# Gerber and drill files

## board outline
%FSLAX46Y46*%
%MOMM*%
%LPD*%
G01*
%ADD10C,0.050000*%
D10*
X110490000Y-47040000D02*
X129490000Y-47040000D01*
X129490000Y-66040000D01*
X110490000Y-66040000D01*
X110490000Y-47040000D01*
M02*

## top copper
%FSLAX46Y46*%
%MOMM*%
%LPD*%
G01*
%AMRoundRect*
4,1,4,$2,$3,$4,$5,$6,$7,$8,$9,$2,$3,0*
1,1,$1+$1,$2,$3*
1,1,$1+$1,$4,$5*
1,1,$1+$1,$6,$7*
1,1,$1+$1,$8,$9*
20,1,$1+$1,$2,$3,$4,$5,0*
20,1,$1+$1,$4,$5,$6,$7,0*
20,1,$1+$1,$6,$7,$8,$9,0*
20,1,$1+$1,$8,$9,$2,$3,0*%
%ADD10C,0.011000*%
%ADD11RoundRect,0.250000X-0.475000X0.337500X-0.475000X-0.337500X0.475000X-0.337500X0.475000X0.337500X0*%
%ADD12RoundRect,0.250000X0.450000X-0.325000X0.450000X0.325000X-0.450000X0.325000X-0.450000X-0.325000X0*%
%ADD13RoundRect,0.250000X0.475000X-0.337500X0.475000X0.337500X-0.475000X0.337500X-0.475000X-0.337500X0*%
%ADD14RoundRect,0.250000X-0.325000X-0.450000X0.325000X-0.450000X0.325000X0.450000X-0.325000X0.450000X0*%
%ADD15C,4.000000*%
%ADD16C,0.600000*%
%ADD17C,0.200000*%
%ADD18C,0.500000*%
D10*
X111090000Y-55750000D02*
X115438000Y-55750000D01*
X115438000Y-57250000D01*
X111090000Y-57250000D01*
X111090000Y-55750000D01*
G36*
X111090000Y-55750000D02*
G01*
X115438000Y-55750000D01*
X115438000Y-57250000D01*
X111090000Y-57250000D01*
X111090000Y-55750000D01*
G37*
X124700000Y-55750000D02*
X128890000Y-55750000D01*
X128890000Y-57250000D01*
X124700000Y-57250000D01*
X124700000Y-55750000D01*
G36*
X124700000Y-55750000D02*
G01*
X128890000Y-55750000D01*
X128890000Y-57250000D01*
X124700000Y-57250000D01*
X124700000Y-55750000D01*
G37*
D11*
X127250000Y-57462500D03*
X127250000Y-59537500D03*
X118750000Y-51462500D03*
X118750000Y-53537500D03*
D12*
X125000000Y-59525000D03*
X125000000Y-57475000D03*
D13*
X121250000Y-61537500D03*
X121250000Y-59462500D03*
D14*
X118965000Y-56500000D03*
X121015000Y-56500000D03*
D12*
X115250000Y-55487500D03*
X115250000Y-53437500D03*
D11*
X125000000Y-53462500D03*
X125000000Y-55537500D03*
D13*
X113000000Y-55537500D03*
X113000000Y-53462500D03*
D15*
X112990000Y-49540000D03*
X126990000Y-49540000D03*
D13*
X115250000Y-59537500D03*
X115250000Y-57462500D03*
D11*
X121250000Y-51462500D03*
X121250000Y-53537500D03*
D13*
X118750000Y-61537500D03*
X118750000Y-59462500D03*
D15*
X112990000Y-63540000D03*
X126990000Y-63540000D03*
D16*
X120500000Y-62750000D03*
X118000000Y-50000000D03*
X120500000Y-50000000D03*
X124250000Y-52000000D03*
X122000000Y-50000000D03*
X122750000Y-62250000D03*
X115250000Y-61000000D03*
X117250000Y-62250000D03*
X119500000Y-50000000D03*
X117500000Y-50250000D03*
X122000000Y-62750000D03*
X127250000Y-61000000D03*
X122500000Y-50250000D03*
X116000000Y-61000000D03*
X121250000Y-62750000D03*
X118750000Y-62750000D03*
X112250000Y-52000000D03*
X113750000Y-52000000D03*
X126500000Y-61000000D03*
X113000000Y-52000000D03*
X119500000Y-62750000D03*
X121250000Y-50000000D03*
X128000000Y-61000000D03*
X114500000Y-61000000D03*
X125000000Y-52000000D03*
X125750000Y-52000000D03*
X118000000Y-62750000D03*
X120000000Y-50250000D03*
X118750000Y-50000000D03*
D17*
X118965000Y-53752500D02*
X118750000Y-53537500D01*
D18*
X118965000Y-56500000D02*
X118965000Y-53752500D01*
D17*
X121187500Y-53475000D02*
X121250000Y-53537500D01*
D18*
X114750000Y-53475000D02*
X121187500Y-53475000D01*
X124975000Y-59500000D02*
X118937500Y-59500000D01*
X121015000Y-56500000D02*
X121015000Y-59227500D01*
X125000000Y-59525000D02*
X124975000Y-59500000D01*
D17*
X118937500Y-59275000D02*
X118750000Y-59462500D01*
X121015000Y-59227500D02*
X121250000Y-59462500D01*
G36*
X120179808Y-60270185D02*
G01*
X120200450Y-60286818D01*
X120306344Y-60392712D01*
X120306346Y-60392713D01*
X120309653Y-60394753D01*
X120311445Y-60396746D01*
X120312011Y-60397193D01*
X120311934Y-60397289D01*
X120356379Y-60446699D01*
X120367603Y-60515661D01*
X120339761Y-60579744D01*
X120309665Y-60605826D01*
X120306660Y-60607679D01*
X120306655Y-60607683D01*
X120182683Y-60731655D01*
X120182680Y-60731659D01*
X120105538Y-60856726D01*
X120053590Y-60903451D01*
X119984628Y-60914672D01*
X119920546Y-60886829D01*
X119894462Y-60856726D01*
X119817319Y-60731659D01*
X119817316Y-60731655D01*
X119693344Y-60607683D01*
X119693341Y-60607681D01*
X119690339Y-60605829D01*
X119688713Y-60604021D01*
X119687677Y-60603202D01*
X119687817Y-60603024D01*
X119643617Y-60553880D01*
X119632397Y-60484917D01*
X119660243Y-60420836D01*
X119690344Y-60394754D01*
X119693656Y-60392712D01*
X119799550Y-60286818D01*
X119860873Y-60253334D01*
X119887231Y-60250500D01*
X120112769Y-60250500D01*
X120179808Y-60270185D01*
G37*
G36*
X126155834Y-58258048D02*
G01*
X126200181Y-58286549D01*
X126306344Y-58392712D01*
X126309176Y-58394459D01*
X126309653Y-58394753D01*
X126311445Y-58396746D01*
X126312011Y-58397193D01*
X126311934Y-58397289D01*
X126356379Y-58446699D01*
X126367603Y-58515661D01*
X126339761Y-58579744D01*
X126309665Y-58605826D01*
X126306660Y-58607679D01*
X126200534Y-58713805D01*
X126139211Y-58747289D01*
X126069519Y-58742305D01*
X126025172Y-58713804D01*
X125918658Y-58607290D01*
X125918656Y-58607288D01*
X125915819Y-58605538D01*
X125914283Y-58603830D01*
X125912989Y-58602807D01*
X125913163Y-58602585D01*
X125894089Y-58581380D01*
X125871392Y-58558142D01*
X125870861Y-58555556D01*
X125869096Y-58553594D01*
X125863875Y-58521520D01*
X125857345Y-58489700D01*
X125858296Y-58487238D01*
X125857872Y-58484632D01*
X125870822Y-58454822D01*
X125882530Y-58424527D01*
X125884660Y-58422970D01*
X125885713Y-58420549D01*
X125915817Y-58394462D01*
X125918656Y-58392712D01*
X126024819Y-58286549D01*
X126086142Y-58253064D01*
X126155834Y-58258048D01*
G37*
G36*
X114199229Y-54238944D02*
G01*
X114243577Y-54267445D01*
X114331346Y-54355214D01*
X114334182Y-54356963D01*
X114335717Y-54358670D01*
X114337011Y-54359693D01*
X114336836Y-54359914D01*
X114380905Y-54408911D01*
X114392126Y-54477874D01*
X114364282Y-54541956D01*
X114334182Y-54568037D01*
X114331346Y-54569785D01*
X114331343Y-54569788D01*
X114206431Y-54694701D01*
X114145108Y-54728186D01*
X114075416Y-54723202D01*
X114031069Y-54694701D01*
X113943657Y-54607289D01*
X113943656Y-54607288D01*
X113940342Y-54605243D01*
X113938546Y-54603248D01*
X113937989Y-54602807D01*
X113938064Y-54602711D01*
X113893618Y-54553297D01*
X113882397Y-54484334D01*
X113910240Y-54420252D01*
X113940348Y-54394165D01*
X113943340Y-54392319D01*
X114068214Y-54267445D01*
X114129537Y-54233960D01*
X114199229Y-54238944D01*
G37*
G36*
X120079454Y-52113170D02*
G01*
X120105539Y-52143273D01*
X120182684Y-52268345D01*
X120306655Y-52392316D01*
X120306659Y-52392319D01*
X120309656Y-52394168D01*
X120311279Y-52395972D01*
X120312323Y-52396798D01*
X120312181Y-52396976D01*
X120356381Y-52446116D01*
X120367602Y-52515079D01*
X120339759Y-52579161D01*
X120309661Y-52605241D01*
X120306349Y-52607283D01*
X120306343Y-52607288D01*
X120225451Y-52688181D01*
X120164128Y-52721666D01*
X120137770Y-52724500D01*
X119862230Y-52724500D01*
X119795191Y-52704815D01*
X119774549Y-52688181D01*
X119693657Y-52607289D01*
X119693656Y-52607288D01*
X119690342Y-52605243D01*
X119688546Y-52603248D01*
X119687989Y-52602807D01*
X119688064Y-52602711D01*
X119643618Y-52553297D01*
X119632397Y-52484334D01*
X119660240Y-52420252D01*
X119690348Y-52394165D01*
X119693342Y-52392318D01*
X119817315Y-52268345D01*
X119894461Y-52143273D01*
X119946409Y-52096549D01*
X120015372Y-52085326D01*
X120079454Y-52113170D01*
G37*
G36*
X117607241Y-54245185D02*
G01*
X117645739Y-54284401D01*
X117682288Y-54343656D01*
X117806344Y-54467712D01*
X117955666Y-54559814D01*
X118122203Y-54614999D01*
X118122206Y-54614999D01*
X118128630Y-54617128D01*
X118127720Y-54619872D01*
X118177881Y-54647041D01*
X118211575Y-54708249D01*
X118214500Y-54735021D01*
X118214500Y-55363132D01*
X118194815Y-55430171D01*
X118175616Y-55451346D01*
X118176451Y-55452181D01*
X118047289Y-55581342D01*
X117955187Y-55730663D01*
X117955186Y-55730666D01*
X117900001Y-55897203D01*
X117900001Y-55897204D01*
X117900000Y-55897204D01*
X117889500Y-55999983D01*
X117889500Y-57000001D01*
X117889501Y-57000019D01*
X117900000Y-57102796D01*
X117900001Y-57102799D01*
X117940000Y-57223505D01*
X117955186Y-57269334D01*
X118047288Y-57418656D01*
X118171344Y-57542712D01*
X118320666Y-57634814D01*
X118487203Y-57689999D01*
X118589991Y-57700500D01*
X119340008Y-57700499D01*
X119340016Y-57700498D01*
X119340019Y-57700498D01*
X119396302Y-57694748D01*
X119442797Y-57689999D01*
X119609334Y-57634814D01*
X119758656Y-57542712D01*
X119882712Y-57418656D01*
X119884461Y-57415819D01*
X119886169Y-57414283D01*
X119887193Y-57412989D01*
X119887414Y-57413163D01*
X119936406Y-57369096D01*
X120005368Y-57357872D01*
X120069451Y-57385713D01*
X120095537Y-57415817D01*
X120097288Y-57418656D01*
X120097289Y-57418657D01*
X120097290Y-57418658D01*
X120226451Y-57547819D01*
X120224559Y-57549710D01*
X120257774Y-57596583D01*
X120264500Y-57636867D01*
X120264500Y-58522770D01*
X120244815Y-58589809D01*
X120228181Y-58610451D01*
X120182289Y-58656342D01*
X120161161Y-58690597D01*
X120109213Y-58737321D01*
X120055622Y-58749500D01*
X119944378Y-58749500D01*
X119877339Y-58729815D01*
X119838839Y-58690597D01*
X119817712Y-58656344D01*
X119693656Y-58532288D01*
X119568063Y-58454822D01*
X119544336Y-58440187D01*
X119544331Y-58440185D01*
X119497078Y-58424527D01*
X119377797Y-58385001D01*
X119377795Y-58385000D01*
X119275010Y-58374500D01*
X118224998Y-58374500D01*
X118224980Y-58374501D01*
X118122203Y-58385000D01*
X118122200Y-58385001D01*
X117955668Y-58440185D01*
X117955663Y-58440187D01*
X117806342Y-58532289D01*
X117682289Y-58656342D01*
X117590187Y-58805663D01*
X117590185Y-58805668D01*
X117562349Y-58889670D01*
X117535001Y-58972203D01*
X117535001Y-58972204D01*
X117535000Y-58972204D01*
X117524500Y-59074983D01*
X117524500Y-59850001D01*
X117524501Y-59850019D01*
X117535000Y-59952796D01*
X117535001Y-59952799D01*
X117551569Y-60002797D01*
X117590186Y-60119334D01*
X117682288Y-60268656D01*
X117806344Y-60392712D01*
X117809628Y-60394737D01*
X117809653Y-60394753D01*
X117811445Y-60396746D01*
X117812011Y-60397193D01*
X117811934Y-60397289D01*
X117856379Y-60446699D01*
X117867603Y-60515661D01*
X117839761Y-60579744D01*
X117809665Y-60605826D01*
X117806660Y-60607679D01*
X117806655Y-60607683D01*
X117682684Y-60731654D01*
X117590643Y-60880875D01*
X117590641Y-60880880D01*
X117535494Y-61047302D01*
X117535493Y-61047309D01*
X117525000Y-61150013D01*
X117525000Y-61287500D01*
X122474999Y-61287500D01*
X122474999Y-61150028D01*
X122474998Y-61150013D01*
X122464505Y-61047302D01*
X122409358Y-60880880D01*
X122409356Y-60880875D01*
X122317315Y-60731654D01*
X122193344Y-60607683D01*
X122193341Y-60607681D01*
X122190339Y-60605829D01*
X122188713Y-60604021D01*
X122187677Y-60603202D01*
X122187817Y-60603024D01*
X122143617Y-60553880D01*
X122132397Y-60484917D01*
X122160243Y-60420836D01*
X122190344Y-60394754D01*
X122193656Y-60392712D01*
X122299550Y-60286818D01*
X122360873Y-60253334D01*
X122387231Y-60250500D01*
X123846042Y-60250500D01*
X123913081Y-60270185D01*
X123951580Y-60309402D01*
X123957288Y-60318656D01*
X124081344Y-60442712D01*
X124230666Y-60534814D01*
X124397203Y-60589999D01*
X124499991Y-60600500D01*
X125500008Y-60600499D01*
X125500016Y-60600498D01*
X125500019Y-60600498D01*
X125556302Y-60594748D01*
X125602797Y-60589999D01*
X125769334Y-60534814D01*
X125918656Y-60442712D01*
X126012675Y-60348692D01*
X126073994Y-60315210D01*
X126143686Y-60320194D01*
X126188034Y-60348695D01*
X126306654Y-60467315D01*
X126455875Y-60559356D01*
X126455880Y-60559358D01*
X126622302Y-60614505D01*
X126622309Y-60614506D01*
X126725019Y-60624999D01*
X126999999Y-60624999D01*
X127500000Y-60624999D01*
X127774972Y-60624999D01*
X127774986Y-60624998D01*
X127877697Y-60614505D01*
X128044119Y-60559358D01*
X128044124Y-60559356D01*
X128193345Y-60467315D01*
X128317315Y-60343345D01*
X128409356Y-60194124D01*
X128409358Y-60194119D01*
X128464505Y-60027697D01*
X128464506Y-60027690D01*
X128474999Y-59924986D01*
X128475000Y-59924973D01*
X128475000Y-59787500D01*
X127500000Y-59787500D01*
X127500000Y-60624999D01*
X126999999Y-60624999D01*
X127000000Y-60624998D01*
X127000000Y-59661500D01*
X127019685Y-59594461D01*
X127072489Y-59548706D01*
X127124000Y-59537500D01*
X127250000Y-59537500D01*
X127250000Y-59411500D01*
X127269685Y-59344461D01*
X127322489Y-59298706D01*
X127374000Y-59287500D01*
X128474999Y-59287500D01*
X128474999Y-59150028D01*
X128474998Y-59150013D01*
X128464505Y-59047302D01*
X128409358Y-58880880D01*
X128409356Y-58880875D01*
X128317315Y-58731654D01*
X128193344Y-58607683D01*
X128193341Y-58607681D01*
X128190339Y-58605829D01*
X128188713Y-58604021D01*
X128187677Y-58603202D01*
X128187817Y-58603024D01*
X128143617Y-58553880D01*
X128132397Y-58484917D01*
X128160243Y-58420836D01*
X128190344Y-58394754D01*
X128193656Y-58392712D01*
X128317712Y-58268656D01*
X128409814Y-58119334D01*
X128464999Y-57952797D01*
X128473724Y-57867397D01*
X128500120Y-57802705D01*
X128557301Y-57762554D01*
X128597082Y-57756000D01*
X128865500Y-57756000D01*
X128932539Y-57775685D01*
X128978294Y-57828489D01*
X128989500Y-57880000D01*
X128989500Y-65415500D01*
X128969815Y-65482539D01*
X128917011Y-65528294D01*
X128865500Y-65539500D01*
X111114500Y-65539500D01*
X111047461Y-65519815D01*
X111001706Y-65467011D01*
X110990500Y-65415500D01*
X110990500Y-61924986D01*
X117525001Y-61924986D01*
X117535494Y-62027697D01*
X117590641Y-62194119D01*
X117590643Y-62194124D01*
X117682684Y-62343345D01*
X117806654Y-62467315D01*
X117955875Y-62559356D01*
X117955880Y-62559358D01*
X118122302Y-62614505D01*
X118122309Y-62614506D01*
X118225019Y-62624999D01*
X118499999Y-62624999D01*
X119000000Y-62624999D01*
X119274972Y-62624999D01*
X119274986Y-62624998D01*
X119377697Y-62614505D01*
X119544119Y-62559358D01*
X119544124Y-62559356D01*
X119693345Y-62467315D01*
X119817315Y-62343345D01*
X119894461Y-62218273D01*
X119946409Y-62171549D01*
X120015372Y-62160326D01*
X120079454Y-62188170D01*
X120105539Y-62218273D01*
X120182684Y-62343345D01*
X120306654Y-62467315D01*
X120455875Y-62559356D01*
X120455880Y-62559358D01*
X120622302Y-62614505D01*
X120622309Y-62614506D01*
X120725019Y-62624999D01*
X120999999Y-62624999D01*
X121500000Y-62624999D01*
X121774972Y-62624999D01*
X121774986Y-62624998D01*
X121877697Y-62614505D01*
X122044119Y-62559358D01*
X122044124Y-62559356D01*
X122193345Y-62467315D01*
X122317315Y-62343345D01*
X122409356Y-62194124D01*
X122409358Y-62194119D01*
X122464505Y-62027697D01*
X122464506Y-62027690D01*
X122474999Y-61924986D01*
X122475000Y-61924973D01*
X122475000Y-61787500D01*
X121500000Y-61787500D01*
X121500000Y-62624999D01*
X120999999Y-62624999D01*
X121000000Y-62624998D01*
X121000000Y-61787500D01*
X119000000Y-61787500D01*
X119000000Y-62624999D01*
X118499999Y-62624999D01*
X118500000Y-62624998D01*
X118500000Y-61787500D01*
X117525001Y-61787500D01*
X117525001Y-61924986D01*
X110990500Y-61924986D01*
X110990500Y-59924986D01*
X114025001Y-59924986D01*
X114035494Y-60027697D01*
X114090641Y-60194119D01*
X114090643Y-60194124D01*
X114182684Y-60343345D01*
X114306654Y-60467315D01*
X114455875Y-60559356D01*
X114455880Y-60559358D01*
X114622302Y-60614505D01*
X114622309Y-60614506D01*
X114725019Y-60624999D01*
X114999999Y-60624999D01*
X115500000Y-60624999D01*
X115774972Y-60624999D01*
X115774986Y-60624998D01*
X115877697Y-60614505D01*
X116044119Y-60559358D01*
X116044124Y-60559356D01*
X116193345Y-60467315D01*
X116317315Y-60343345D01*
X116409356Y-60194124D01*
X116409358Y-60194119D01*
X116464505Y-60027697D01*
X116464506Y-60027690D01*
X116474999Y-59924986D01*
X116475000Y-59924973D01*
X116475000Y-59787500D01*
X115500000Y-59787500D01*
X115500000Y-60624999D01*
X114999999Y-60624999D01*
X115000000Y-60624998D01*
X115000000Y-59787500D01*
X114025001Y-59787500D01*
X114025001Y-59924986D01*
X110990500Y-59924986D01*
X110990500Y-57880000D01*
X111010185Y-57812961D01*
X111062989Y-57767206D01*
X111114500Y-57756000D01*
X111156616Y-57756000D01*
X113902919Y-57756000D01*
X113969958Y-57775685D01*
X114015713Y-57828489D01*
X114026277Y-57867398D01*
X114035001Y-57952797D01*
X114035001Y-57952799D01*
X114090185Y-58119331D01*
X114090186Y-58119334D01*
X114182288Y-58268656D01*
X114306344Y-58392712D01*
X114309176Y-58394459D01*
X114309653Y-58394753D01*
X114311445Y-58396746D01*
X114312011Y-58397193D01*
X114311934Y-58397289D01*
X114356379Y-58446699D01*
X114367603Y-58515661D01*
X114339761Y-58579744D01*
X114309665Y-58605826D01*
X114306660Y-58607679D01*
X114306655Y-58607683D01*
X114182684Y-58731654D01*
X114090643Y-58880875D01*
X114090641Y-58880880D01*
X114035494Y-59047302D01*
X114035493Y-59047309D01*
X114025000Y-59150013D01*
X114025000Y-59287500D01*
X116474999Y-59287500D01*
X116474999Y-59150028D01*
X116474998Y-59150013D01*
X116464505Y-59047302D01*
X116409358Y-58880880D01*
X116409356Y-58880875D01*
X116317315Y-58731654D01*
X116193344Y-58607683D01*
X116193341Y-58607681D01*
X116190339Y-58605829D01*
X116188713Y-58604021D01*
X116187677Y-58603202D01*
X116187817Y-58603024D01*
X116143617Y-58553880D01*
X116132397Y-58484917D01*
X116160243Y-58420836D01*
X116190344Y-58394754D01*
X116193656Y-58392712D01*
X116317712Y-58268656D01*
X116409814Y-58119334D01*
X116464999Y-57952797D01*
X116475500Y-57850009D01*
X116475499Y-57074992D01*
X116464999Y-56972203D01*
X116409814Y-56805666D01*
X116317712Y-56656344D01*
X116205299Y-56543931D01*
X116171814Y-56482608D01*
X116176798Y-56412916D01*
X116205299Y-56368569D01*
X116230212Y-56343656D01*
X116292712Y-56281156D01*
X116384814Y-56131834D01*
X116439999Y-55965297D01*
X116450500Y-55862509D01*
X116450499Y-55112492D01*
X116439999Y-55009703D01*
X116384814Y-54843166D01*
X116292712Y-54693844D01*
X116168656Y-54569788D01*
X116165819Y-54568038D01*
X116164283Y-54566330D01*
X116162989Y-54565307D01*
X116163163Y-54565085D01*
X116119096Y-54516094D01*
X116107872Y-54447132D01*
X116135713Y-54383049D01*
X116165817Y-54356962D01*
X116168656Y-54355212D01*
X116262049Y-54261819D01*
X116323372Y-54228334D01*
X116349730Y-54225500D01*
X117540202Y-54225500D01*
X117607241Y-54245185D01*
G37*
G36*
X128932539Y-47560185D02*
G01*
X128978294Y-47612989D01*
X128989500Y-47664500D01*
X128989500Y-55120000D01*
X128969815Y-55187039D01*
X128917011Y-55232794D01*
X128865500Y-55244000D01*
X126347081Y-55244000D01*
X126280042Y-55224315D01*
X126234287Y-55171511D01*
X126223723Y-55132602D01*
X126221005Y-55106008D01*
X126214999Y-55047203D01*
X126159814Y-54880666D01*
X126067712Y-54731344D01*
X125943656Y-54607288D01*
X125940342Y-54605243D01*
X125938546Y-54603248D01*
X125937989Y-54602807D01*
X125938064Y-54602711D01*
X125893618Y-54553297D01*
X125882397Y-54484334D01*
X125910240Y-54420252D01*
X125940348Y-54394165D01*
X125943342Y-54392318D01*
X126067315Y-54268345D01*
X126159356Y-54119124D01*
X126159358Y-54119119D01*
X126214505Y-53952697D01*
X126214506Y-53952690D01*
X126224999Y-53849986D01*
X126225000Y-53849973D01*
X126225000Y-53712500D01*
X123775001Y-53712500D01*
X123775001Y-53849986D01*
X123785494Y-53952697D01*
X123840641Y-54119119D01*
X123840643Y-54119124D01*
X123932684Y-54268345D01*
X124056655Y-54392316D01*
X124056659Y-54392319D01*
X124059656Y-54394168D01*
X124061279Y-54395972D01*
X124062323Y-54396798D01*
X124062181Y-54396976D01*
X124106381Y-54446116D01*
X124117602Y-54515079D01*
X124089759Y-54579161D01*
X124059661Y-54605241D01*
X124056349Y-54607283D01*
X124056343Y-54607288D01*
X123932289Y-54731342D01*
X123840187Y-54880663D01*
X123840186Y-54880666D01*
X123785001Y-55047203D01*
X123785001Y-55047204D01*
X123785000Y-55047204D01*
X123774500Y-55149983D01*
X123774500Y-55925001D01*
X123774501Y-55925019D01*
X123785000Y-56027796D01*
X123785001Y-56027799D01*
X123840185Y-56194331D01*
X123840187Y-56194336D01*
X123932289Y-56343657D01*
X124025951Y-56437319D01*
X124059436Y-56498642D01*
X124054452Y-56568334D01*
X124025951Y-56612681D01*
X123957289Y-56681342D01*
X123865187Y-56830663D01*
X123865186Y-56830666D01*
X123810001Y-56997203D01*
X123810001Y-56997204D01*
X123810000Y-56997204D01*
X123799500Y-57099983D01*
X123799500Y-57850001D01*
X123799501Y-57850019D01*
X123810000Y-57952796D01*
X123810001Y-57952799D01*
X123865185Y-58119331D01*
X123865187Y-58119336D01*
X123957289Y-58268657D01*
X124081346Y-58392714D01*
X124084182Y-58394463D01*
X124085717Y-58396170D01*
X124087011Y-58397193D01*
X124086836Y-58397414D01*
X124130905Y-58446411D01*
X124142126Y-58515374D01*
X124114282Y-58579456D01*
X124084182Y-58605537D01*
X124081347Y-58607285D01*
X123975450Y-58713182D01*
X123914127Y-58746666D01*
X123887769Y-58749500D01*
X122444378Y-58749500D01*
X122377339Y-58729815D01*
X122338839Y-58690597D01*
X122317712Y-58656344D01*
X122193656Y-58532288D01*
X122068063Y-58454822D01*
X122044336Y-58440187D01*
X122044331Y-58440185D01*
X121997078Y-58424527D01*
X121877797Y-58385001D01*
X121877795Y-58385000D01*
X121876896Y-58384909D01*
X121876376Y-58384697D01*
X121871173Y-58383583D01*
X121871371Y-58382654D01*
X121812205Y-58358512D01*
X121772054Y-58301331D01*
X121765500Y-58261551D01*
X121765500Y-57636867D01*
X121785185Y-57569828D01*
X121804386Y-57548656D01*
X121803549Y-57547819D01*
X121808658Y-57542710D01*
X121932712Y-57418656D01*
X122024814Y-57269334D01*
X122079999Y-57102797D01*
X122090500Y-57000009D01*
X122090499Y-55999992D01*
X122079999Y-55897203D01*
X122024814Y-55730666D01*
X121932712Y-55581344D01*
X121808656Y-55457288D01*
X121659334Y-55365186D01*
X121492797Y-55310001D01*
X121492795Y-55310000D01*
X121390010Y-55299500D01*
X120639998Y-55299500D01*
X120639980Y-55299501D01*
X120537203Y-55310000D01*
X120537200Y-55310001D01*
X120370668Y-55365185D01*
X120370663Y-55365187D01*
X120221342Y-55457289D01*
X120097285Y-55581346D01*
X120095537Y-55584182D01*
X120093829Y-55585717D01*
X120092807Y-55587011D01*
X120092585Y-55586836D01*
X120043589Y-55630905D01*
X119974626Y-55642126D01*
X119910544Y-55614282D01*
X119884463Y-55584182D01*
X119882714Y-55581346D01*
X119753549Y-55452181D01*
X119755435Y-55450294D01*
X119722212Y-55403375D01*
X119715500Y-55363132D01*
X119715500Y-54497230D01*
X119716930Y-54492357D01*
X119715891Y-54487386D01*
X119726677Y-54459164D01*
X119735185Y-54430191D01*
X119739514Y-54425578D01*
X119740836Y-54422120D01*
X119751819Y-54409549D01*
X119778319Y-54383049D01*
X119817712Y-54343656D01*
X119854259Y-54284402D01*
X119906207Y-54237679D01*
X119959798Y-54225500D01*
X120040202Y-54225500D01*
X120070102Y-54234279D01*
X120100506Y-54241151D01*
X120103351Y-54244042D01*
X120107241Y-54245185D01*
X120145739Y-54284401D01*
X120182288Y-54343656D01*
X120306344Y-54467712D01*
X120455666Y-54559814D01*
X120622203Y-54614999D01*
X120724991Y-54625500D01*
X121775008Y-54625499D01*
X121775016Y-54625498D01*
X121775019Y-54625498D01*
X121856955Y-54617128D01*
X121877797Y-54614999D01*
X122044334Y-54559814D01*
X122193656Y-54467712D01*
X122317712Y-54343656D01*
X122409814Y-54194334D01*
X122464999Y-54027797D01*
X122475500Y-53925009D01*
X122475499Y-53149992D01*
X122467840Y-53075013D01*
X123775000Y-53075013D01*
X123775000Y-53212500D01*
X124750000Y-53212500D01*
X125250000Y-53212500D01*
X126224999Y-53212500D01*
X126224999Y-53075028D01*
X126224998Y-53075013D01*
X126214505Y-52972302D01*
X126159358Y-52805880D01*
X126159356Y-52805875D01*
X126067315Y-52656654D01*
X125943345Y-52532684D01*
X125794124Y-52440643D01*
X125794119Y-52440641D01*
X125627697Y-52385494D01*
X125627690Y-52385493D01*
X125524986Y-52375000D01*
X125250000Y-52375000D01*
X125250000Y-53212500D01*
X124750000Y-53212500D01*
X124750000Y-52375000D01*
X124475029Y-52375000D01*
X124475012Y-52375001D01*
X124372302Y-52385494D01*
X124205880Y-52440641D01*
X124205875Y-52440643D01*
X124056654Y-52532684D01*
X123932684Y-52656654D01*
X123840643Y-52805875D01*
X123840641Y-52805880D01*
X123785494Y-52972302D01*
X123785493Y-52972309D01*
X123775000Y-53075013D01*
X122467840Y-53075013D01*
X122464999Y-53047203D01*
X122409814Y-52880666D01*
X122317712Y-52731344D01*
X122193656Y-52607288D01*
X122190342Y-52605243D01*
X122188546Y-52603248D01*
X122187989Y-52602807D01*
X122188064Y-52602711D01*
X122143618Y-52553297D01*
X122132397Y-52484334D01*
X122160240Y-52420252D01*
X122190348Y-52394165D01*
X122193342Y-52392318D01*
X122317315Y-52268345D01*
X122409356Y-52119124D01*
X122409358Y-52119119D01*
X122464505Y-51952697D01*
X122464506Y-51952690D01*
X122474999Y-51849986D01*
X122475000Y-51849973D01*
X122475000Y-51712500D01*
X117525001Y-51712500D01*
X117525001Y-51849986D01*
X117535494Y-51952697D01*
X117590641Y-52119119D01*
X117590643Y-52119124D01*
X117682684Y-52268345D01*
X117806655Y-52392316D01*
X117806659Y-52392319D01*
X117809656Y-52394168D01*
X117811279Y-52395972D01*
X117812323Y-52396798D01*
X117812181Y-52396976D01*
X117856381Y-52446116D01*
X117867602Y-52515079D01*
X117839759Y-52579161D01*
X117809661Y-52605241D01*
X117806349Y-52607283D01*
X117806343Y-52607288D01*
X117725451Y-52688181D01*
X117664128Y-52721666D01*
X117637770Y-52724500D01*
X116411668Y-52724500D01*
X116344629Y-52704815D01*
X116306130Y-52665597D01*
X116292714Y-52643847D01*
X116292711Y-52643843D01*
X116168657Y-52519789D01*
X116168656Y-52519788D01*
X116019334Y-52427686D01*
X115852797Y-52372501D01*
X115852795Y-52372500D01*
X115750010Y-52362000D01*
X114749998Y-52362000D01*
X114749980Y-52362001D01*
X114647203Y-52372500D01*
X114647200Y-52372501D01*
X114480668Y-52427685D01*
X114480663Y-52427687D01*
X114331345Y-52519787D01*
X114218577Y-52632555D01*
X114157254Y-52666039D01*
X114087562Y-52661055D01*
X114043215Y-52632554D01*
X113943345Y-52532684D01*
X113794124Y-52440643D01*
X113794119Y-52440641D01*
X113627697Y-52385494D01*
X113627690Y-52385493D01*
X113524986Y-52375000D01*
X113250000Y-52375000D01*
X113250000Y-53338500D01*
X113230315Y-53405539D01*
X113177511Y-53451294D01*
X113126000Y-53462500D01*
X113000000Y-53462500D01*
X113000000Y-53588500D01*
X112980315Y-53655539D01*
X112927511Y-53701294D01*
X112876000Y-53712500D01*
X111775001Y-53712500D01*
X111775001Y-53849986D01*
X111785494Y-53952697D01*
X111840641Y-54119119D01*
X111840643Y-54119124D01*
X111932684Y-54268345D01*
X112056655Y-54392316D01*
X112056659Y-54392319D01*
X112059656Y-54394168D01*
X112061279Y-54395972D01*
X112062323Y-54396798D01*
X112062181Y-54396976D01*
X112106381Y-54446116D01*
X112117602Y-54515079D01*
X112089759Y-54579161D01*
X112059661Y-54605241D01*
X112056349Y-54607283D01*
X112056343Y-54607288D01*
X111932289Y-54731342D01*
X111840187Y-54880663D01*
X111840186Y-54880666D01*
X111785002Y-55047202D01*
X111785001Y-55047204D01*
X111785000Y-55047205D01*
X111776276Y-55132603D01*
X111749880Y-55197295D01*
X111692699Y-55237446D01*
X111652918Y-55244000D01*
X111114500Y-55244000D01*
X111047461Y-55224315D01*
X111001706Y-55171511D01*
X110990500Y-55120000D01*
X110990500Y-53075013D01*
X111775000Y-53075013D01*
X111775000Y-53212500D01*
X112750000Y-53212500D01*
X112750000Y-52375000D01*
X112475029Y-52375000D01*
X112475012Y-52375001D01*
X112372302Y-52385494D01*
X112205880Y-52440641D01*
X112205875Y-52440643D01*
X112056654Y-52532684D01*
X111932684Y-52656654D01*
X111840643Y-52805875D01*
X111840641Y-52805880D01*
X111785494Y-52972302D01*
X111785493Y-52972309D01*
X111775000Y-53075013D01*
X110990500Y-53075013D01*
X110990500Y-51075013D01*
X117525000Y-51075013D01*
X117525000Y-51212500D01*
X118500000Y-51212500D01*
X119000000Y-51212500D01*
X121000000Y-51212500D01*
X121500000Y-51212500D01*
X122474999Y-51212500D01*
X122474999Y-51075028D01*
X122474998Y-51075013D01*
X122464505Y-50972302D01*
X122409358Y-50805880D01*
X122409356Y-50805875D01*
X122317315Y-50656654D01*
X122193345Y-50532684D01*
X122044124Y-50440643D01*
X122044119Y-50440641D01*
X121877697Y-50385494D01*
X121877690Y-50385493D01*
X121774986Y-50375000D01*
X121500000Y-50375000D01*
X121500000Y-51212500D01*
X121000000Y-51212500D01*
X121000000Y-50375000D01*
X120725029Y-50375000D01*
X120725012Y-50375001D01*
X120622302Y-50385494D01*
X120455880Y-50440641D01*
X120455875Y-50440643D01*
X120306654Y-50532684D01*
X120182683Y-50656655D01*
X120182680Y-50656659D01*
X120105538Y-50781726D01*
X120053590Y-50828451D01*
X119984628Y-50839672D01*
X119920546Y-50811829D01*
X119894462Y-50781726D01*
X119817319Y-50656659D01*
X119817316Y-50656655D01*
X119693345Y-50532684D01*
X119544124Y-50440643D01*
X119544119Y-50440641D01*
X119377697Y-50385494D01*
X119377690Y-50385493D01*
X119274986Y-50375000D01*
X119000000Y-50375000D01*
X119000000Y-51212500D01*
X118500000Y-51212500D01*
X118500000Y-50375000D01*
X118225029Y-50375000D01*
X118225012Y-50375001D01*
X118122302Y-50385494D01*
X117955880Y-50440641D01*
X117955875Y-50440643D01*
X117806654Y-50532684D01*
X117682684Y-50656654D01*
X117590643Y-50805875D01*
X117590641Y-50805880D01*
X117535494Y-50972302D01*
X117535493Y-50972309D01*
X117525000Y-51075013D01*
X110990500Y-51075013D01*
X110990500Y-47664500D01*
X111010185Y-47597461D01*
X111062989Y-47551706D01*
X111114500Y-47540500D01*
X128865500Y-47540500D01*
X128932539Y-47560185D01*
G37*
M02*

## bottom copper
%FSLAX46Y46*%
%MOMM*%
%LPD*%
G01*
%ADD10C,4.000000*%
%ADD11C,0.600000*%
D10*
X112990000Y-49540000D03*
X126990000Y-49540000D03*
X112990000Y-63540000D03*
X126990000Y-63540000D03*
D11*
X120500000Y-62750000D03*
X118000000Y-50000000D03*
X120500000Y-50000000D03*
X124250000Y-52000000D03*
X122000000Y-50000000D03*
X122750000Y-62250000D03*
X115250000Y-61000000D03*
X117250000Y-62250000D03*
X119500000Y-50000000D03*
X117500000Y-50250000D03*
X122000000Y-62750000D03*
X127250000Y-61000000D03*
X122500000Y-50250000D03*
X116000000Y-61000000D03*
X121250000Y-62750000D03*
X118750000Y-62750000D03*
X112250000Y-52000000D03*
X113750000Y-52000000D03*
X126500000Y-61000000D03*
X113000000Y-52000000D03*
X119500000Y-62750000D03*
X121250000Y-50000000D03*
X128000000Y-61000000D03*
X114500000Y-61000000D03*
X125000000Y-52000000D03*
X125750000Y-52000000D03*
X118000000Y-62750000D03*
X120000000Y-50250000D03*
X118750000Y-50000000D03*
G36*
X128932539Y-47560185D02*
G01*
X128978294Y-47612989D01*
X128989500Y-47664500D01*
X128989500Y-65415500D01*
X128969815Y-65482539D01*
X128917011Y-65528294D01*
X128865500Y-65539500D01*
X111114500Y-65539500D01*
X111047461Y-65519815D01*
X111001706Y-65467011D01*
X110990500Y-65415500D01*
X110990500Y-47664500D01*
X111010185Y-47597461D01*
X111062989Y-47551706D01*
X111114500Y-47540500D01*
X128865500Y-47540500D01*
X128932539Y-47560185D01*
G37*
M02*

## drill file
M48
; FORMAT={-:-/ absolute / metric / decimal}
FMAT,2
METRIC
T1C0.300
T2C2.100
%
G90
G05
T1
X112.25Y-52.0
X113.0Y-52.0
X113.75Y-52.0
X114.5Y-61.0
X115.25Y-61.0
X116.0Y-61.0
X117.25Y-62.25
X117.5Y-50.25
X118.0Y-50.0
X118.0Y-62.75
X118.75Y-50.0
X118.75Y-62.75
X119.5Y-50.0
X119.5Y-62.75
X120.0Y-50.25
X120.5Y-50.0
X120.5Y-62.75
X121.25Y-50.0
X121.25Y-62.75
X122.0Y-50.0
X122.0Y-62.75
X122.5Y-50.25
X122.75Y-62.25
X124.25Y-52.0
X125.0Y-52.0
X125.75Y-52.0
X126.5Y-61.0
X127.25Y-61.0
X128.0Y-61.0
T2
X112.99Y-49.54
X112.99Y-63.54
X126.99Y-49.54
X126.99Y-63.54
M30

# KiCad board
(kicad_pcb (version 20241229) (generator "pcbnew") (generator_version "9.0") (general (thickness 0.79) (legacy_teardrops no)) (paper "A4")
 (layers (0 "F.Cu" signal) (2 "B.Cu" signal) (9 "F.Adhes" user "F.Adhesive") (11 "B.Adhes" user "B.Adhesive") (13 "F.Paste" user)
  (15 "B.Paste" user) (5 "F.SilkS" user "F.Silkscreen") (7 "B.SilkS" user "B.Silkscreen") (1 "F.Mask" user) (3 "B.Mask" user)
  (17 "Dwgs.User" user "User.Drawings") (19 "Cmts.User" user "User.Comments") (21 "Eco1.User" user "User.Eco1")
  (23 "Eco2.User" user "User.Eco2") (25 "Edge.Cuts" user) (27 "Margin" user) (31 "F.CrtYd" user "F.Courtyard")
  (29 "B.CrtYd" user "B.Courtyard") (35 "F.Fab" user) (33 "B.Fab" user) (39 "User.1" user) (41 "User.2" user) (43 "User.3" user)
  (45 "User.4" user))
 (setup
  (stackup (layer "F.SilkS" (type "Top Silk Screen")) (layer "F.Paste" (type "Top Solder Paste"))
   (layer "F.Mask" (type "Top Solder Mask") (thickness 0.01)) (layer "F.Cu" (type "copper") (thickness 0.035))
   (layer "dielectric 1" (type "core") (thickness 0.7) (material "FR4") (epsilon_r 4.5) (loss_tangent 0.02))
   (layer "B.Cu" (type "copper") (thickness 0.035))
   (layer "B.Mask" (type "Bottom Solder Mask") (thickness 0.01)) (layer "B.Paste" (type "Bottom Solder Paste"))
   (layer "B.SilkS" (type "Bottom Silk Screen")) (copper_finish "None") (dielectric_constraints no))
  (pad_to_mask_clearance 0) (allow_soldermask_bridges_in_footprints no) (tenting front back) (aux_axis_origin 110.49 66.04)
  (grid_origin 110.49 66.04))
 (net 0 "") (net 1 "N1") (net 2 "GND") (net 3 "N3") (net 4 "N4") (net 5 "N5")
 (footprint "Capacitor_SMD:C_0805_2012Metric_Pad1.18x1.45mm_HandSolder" (layer "F.Cu") (at 127.25 58.5 -90)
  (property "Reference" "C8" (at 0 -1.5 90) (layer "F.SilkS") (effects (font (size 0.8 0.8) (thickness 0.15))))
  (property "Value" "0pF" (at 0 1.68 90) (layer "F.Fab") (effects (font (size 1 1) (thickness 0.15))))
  (pad "1" smd roundrect (at -1.0375 0 270) (size 1.175 1.45) (layers "F.Cu" "F.Mask" "F.Paste") (roundrect_rratio 0.212766) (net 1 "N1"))
  (pad "2" smd roundrect (at 1.0375 0 270) (size 1.175 1.45) (layers "F.Cu" "F.Mask" "F.Paste") (roundrect_rratio 0.212766) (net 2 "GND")))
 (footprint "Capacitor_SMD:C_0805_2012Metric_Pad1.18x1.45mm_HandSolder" (layer "F.Cu") (at 118.75 52.5 -90)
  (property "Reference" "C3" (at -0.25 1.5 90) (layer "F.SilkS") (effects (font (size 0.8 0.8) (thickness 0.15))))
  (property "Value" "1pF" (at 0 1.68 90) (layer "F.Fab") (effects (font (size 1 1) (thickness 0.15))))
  (pad "1" smd roundrect (at -1.0375 0 270) (size 1.175 1.45) (layers "F.Cu" "F.Mask" "F.Paste") (roundrect_rratio 0.212766) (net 2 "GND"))
  (pad "2" smd roundrect (at 1.0375 0 270) (size 1.175 1.45) (layers "F.Cu" "F.Mask" "F.Paste") (roundrect_rratio 0.212766) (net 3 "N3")))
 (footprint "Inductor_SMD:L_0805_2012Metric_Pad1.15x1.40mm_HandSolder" (layer "F.Cu") (at 125 58.5 90)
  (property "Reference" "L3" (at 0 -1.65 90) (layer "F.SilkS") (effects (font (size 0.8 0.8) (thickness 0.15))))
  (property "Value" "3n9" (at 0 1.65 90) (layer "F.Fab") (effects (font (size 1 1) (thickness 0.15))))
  (pad "1" smd roundrect (at -1.025 0 90) (size 1.15 1.4) (layers "F.Cu" "F.Mask" "F.Paste") (roundrect_rratio 0.217391) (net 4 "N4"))
  (pad "2" smd roundrect (at 1.025 0 90) (size 1.15 1.4) (layers "F.Cu" "F.Mask" "F.Paste") (roundrect_rratio 0.217391) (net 1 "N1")))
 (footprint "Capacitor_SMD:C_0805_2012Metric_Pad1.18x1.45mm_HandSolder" (layer "F.Cu") (at 121.25 60.5 90)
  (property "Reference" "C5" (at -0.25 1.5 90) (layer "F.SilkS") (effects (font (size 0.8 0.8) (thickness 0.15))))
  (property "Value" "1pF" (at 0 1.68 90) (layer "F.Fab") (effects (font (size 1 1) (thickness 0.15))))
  (pad "1" smd roundrect (at -1.0375 0 90) (size 1.175 1.45) (layers "F.Cu" "F.Mask" "F.Paste") (roundrect_rratio 0.212766) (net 2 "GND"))
  (pad "2" smd roundrect (at 1.0375 0 90) (size 1.175 1.45) (layers "F.Cu" "F.Mask" "F.Paste") (roundrect_rratio 0.212766) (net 4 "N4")))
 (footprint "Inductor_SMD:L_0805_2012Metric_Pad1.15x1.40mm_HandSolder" (layer "F.Cu") (at 119.99 56.5)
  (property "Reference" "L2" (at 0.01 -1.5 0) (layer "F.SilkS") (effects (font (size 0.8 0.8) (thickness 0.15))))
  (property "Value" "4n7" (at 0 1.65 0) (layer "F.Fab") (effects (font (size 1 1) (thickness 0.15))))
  (pad "1" smd roundrect (at -1.025 0) (size 1.15 1.4) (layers "F.Cu" "F.Mask" "F.Paste") (roundrect_rratio 0.217391) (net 3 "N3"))
  (pad "2" smd roundrect (at 1.025 0) (size 1.15 1.4) (layers "F.Cu" "F.Mask" "F.Paste") (roundrect_rratio 0.217391) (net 4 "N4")))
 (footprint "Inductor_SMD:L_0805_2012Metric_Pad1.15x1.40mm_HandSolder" (layer "F.Cu") (at 115.25 54.4625 90)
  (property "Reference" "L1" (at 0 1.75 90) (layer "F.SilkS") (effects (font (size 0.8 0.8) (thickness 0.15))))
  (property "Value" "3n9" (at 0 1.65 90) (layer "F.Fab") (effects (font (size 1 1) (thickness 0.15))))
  (pad "1" smd roundrect (at -1.025 0 90) (size 1.15 1.4) (layers "F.Cu" "F.Mask" "F.Paste") (roundrect_rratio 0.217391) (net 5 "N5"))
  (pad "2" smd roundrect (at 1.025 0 90) (size 1.15 1.4) (layers "F.Cu" "F.Mask" "F.Paste") (roundrect_rratio 0.217391) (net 3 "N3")))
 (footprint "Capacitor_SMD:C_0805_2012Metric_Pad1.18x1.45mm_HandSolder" (layer "F.Cu") (at 125 54.5 -90)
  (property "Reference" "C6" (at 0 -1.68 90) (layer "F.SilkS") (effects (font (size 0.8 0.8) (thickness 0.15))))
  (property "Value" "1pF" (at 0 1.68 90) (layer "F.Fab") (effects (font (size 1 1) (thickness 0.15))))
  (pad "1" smd roundrect (at -1.0375 0 270) (size 1.175 1.45) (layers "F.Cu" "F.Mask" "F.Paste") (roundrect_rratio 0.212766) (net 2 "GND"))
  (pad "2" smd roundrect (at 1.0375 0 270) (size 1.175 1.45) (layers "F.Cu" "F.Mask" "F.Paste") (roundrect_rratio 0.212766) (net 1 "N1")))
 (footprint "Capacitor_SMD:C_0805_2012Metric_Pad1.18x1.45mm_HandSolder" (layer "F.Cu") (at 113 54.5 90)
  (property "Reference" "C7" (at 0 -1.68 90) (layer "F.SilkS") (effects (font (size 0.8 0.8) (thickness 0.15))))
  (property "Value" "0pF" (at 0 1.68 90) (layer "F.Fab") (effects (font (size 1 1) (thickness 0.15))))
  (pad "1" smd roundrect (at -1.0375 0 90) (size 1.175 1.45) (layers "F.Cu" "F.Mask" "F.Paste") (roundrect_rratio 0.212766) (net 5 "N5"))
  (pad "2" smd roundrect (at 1.0375 0 90) (size 1.175 1.45) (layers "F.Cu" "F.Mask" "F.Paste") (roundrect_rratio 0.212766) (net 2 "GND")))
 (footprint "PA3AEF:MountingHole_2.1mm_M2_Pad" (layer "F.Cu") (at 112.99 49.54)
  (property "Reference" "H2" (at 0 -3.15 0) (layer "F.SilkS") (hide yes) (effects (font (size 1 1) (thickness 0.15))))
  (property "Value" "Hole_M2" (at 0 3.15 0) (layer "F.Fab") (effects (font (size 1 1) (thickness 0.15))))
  (pad "1" thru_hole circle (at 0 0) (size 4 4) (drill 2.1) (layers "*.Cu" "*.Mask") (remove_unused_layers no) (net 2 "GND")
   (zone_connect 2)))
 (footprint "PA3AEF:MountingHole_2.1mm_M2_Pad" (layer "F.Cu") (at 126.99 49.54)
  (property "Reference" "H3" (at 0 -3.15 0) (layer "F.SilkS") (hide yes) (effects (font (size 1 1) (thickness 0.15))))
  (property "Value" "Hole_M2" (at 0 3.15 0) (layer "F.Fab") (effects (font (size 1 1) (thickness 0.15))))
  (pad "1" thru_hole circle (at 0 0) (size 4 4) (drill 2.1) (layers "*.Cu" "*.Mask") (remove_unused_layers no) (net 2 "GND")
   (zone_connect 2)))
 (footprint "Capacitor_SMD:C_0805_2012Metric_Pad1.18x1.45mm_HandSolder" (layer "F.Cu") (at 115.25 58.5 90)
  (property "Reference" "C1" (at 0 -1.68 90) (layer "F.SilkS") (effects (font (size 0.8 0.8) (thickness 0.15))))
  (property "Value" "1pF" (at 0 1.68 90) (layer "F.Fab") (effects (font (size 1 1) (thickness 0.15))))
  (pad "1" smd roundrect (at -1.0375 0 90) (size 1.175 1.45) (layers "F.Cu" "F.Mask" "F.Paste") (roundrect_rratio 0.212766) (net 2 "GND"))
  (pad "2" smd roundrect (at 1.0375 0 90) (size 1.175 1.45) (layers "F.Cu" "F.Mask" "F.Paste") (roundrect_rratio 0.212766) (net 5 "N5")))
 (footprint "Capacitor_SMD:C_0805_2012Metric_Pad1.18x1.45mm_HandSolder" (layer "F.Cu") (at 121.25 52.5 -90)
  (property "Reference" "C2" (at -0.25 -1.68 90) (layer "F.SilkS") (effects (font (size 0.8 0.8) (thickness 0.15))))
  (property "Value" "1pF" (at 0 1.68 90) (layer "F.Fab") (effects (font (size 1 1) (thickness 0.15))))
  (pad "1" smd roundrect (at -1.0375 0 270) (size 1.175 1.45) (layers "F.Cu" "F.Mask" "F.Paste") (roundrect_rratio 0.212766) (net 2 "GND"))
  (pad "2" smd roundrect (at 1.0375 0 270) (size 1.175 1.45) (layers "F.Cu" "F.Mask" "F.Paste") (roundrect_rratio 0.212766) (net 3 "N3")))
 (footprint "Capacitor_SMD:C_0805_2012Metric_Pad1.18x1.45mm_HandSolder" (layer "F.Cu") (at 118.75 60.5 90)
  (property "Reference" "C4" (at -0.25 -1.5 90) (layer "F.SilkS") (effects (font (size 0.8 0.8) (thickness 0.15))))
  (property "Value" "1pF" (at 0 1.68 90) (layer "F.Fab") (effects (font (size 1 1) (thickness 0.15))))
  (pad "1" smd roundrect (at -1.0375 0 90) (size 1.175 1.45) (layers "F.Cu" "F.Mask" "F.Paste") (roundrect_rratio 0.212766) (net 2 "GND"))
  (pad "2" smd roundrect (at 1.0375 0 90) (size 1.175 1.45) (layers "F.Cu" "F.Mask" "F.Paste") (roundrect_rratio 0.212766) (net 4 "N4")))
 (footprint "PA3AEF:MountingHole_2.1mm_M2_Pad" (layer "F.Cu") (at 112.99 63.54)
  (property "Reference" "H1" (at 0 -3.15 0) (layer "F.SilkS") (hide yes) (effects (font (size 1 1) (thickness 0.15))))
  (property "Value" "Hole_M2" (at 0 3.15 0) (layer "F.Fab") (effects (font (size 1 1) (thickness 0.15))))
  (pad "1" thru_hole circle (at 0 0) (size 4 4) (drill 2.1) (layers "*.Cu" "*.Mask") (remove_unused_layers no) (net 2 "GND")
   (zone_connect 2)))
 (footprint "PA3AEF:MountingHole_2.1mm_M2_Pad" (layer "F.Cu") (at 126.99 63.54)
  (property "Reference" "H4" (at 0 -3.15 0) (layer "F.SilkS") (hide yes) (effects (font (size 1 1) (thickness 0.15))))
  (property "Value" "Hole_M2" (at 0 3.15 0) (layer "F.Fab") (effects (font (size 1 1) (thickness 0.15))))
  (pad "1" thru_hole circle (at 0 0) (size 4 4) (drill 2.1) (layers "*.Cu" "*.Mask") (remove_unused_layers no) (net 2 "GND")
   (zone_connect 2)))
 (gr_rect (start 111.09 55.75) (end 115.438 57.25) (stroke (width 0.011) (type solid)) (fill yes) (layer "F.Cu") (net 5))
 (gr_rect (start 124.7 55.75) (end 128.89 57.25) (stroke (width 0.011) (type solid)) (fill yes) (layer "F.Cu") (net 1))
 (gr_rect (start 110.49 47.04) (end 129.49 66.04) (stroke (width 0.05) (type solid)) (fill no) (layer "Edge.Cuts"))
 (via (at 120.5 62.75) (size 0.6) (drill 0.3) (layers "F.Cu" "B.Cu") (free yes) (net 2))
 (via (at 118 50) (size 0.6) (drill 0.3) (layers "F.Cu" "B.Cu") (free yes) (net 2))
 (via (at 120.5 50) (size 0.6) (drill 0.3) (layers "F.Cu" "B.Cu") (free yes) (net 2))
 (via (at 124.25 52) (size 0.6) (drill 0.3) (layers "F.Cu" "B.Cu") (free yes) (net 2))
 (via (at 122 50) (size 0.6) (drill 0.3) (layers "F.Cu" "B.Cu") (free yes) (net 2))
 (via (at 122.75 62.25) (size 0.6) (drill 0.3) (layers "F.Cu" "B.Cu") (free yes) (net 2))
 (via (at 115.25 61) (size 0.6) (drill 0.3) (layers "F.Cu" "B.Cu") (free yes) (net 2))
 (via (at 117.25 62.25) (size 0.6) (drill 0.3) (layers "F.Cu" "B.Cu") (free yes) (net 2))
 (via (at 119.5 50) (size 0.6) (drill 0.3) (layers "F.Cu" "B.Cu") (free yes) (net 2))
 (via (at 117.5 50.25) (size 0.6) (drill 0.3) (layers "F.Cu" "B.Cu") (free yes) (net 2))
 (via (at 122 62.75) (size 0.6) (drill 0.3) (layers "F.Cu" "B.Cu") (free yes) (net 2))
 (via (at 127.25 61) (size 0.6) (drill 0.3) (layers "F.Cu" "B.Cu") (free yes) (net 2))
 (via (at 122.5 50.25) (size 0.6) (drill 0.3) (layers "F.Cu" "B.Cu") (free yes) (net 2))
 (via (at 116 61) (size 0.6) (drill 0.3) (layers "F.Cu" "B.Cu") (free yes) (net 2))
 (via (at 121.25 62.75) (size 0.6) (drill 0.3) (layers "F.Cu" "B.Cu") (free yes) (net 2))
 (via (at 118.75 62.75) (size 0.6) (drill 0.3) (layers "F.Cu" "B.Cu") (free yes) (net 2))
 (via (at 112.25 52) (size 0.6) (drill 0.3) (layers "F.Cu" "B.Cu") (free yes) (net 2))
 (via (at 113.75 52) (size 0.6) (drill 0.3) (layers "F.Cu" "B.Cu") (free yes) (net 2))
 (via (at 126.5 61) (size 0.6) (drill 0.3) (layers "F.Cu" "B.Cu") (free yes) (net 2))
 (via (at 113 52) (size 0.6) (drill 0.3) (layers "F.Cu" "B.Cu") (free yes) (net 2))
 (via (at 119.5 62.75) (size 0.6) (drill 0.3) (layers "F.Cu" "B.Cu") (free yes) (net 2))
 (via (at 121.25 50) (size 0.6) (drill 0.3) (layers "F.Cu" "B.Cu") (free yes) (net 2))
 (via (at 128 61) (size 0.6) (drill 0.3) (layers "F.Cu" "B.Cu") (free yes) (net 2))
 (via (at 114.5 61) (size 0.6) (drill 0.3) (layers "F.Cu" "B.Cu") (free yes) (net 2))
 (via (at 125 52) (size 0.6) (drill 0.3) (layers "F.Cu" "B.Cu") (free yes) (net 2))
 (via (at 125.75 52) (size 0.6) (drill 0.3) (layers "F.Cu" "B.Cu") (free yes) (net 2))
 (via (at 118 62.75) (size 0.6) (drill 0.3) (layers "F.Cu" "B.Cu") (free yes) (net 2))
 (via (at 120 50.25) (size 0.6) (drill 0.3) (layers "F.Cu" "B.Cu") (free yes) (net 2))
 (via (at 118.75 50) (size 0.6) (drill 0.3) (layers "F.Cu" "B.Cu") (free yes) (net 2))
 (segment (start 118.965 53.7525) (end 118.75 53.5375) (width 0.2) (layer "F.Cu") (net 3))
 (segment (start 118.965 56.5) (end 118.965 53.7525) (width 0.5) (layer "F.Cu") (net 3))
 (segment (start 121.1875 53.475) (end 121.25 53.5375) (width 0.2) (layer "F.Cu") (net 3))
 (segment (start 114.75 53.475) (end 121.1875 53.475) (width 0.5) (layer "F.Cu") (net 3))
 (segment (start 124.975 59.5) (end 118.9375 59.5) (width 0.5) (layer "F.Cu") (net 4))
 (segment (start 121.015 56.5) (end 121.015 59.2275) (width 0.5) (layer "F.Cu") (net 4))
 (segment (start 125 59.525) (end 124.975 59.5) (width 0.5) (layer "F.Cu") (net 4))
 (segment (start 118.9375 59.275) (end 118.75 59.4625) (width 0.2) (layer "F.Cu") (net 4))
 (segment (start 121.015 59.2275) (end 121.25 59.4625) (width 0.2) (layer "F.Cu") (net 4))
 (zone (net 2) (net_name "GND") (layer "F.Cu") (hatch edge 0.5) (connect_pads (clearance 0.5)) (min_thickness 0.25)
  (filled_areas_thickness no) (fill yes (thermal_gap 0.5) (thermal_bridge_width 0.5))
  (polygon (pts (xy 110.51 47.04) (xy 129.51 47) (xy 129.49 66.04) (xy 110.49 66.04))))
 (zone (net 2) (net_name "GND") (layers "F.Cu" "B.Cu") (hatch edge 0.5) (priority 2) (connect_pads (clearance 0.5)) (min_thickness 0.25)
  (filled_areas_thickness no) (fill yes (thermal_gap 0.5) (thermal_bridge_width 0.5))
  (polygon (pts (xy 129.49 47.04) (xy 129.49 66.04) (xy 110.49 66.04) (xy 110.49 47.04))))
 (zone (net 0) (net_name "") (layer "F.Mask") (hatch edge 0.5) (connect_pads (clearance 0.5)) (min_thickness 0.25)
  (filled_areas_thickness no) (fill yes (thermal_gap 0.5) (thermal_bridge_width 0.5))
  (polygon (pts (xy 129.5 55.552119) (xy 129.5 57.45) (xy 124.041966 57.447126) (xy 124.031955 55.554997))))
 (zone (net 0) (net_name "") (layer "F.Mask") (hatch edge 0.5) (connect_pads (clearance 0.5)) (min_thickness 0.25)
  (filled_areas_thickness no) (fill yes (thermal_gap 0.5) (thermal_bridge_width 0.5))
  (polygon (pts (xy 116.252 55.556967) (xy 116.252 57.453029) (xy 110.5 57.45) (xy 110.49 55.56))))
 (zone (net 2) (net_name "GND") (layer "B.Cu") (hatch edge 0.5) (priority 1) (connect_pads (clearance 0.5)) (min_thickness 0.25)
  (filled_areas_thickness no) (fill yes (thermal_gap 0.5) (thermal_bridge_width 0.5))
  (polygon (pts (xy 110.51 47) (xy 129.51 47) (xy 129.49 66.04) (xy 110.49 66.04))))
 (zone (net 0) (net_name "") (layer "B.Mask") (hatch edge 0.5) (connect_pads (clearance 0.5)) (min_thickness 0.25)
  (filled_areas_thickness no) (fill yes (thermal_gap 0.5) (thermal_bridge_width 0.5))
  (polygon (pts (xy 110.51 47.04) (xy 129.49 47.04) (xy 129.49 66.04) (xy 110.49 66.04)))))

